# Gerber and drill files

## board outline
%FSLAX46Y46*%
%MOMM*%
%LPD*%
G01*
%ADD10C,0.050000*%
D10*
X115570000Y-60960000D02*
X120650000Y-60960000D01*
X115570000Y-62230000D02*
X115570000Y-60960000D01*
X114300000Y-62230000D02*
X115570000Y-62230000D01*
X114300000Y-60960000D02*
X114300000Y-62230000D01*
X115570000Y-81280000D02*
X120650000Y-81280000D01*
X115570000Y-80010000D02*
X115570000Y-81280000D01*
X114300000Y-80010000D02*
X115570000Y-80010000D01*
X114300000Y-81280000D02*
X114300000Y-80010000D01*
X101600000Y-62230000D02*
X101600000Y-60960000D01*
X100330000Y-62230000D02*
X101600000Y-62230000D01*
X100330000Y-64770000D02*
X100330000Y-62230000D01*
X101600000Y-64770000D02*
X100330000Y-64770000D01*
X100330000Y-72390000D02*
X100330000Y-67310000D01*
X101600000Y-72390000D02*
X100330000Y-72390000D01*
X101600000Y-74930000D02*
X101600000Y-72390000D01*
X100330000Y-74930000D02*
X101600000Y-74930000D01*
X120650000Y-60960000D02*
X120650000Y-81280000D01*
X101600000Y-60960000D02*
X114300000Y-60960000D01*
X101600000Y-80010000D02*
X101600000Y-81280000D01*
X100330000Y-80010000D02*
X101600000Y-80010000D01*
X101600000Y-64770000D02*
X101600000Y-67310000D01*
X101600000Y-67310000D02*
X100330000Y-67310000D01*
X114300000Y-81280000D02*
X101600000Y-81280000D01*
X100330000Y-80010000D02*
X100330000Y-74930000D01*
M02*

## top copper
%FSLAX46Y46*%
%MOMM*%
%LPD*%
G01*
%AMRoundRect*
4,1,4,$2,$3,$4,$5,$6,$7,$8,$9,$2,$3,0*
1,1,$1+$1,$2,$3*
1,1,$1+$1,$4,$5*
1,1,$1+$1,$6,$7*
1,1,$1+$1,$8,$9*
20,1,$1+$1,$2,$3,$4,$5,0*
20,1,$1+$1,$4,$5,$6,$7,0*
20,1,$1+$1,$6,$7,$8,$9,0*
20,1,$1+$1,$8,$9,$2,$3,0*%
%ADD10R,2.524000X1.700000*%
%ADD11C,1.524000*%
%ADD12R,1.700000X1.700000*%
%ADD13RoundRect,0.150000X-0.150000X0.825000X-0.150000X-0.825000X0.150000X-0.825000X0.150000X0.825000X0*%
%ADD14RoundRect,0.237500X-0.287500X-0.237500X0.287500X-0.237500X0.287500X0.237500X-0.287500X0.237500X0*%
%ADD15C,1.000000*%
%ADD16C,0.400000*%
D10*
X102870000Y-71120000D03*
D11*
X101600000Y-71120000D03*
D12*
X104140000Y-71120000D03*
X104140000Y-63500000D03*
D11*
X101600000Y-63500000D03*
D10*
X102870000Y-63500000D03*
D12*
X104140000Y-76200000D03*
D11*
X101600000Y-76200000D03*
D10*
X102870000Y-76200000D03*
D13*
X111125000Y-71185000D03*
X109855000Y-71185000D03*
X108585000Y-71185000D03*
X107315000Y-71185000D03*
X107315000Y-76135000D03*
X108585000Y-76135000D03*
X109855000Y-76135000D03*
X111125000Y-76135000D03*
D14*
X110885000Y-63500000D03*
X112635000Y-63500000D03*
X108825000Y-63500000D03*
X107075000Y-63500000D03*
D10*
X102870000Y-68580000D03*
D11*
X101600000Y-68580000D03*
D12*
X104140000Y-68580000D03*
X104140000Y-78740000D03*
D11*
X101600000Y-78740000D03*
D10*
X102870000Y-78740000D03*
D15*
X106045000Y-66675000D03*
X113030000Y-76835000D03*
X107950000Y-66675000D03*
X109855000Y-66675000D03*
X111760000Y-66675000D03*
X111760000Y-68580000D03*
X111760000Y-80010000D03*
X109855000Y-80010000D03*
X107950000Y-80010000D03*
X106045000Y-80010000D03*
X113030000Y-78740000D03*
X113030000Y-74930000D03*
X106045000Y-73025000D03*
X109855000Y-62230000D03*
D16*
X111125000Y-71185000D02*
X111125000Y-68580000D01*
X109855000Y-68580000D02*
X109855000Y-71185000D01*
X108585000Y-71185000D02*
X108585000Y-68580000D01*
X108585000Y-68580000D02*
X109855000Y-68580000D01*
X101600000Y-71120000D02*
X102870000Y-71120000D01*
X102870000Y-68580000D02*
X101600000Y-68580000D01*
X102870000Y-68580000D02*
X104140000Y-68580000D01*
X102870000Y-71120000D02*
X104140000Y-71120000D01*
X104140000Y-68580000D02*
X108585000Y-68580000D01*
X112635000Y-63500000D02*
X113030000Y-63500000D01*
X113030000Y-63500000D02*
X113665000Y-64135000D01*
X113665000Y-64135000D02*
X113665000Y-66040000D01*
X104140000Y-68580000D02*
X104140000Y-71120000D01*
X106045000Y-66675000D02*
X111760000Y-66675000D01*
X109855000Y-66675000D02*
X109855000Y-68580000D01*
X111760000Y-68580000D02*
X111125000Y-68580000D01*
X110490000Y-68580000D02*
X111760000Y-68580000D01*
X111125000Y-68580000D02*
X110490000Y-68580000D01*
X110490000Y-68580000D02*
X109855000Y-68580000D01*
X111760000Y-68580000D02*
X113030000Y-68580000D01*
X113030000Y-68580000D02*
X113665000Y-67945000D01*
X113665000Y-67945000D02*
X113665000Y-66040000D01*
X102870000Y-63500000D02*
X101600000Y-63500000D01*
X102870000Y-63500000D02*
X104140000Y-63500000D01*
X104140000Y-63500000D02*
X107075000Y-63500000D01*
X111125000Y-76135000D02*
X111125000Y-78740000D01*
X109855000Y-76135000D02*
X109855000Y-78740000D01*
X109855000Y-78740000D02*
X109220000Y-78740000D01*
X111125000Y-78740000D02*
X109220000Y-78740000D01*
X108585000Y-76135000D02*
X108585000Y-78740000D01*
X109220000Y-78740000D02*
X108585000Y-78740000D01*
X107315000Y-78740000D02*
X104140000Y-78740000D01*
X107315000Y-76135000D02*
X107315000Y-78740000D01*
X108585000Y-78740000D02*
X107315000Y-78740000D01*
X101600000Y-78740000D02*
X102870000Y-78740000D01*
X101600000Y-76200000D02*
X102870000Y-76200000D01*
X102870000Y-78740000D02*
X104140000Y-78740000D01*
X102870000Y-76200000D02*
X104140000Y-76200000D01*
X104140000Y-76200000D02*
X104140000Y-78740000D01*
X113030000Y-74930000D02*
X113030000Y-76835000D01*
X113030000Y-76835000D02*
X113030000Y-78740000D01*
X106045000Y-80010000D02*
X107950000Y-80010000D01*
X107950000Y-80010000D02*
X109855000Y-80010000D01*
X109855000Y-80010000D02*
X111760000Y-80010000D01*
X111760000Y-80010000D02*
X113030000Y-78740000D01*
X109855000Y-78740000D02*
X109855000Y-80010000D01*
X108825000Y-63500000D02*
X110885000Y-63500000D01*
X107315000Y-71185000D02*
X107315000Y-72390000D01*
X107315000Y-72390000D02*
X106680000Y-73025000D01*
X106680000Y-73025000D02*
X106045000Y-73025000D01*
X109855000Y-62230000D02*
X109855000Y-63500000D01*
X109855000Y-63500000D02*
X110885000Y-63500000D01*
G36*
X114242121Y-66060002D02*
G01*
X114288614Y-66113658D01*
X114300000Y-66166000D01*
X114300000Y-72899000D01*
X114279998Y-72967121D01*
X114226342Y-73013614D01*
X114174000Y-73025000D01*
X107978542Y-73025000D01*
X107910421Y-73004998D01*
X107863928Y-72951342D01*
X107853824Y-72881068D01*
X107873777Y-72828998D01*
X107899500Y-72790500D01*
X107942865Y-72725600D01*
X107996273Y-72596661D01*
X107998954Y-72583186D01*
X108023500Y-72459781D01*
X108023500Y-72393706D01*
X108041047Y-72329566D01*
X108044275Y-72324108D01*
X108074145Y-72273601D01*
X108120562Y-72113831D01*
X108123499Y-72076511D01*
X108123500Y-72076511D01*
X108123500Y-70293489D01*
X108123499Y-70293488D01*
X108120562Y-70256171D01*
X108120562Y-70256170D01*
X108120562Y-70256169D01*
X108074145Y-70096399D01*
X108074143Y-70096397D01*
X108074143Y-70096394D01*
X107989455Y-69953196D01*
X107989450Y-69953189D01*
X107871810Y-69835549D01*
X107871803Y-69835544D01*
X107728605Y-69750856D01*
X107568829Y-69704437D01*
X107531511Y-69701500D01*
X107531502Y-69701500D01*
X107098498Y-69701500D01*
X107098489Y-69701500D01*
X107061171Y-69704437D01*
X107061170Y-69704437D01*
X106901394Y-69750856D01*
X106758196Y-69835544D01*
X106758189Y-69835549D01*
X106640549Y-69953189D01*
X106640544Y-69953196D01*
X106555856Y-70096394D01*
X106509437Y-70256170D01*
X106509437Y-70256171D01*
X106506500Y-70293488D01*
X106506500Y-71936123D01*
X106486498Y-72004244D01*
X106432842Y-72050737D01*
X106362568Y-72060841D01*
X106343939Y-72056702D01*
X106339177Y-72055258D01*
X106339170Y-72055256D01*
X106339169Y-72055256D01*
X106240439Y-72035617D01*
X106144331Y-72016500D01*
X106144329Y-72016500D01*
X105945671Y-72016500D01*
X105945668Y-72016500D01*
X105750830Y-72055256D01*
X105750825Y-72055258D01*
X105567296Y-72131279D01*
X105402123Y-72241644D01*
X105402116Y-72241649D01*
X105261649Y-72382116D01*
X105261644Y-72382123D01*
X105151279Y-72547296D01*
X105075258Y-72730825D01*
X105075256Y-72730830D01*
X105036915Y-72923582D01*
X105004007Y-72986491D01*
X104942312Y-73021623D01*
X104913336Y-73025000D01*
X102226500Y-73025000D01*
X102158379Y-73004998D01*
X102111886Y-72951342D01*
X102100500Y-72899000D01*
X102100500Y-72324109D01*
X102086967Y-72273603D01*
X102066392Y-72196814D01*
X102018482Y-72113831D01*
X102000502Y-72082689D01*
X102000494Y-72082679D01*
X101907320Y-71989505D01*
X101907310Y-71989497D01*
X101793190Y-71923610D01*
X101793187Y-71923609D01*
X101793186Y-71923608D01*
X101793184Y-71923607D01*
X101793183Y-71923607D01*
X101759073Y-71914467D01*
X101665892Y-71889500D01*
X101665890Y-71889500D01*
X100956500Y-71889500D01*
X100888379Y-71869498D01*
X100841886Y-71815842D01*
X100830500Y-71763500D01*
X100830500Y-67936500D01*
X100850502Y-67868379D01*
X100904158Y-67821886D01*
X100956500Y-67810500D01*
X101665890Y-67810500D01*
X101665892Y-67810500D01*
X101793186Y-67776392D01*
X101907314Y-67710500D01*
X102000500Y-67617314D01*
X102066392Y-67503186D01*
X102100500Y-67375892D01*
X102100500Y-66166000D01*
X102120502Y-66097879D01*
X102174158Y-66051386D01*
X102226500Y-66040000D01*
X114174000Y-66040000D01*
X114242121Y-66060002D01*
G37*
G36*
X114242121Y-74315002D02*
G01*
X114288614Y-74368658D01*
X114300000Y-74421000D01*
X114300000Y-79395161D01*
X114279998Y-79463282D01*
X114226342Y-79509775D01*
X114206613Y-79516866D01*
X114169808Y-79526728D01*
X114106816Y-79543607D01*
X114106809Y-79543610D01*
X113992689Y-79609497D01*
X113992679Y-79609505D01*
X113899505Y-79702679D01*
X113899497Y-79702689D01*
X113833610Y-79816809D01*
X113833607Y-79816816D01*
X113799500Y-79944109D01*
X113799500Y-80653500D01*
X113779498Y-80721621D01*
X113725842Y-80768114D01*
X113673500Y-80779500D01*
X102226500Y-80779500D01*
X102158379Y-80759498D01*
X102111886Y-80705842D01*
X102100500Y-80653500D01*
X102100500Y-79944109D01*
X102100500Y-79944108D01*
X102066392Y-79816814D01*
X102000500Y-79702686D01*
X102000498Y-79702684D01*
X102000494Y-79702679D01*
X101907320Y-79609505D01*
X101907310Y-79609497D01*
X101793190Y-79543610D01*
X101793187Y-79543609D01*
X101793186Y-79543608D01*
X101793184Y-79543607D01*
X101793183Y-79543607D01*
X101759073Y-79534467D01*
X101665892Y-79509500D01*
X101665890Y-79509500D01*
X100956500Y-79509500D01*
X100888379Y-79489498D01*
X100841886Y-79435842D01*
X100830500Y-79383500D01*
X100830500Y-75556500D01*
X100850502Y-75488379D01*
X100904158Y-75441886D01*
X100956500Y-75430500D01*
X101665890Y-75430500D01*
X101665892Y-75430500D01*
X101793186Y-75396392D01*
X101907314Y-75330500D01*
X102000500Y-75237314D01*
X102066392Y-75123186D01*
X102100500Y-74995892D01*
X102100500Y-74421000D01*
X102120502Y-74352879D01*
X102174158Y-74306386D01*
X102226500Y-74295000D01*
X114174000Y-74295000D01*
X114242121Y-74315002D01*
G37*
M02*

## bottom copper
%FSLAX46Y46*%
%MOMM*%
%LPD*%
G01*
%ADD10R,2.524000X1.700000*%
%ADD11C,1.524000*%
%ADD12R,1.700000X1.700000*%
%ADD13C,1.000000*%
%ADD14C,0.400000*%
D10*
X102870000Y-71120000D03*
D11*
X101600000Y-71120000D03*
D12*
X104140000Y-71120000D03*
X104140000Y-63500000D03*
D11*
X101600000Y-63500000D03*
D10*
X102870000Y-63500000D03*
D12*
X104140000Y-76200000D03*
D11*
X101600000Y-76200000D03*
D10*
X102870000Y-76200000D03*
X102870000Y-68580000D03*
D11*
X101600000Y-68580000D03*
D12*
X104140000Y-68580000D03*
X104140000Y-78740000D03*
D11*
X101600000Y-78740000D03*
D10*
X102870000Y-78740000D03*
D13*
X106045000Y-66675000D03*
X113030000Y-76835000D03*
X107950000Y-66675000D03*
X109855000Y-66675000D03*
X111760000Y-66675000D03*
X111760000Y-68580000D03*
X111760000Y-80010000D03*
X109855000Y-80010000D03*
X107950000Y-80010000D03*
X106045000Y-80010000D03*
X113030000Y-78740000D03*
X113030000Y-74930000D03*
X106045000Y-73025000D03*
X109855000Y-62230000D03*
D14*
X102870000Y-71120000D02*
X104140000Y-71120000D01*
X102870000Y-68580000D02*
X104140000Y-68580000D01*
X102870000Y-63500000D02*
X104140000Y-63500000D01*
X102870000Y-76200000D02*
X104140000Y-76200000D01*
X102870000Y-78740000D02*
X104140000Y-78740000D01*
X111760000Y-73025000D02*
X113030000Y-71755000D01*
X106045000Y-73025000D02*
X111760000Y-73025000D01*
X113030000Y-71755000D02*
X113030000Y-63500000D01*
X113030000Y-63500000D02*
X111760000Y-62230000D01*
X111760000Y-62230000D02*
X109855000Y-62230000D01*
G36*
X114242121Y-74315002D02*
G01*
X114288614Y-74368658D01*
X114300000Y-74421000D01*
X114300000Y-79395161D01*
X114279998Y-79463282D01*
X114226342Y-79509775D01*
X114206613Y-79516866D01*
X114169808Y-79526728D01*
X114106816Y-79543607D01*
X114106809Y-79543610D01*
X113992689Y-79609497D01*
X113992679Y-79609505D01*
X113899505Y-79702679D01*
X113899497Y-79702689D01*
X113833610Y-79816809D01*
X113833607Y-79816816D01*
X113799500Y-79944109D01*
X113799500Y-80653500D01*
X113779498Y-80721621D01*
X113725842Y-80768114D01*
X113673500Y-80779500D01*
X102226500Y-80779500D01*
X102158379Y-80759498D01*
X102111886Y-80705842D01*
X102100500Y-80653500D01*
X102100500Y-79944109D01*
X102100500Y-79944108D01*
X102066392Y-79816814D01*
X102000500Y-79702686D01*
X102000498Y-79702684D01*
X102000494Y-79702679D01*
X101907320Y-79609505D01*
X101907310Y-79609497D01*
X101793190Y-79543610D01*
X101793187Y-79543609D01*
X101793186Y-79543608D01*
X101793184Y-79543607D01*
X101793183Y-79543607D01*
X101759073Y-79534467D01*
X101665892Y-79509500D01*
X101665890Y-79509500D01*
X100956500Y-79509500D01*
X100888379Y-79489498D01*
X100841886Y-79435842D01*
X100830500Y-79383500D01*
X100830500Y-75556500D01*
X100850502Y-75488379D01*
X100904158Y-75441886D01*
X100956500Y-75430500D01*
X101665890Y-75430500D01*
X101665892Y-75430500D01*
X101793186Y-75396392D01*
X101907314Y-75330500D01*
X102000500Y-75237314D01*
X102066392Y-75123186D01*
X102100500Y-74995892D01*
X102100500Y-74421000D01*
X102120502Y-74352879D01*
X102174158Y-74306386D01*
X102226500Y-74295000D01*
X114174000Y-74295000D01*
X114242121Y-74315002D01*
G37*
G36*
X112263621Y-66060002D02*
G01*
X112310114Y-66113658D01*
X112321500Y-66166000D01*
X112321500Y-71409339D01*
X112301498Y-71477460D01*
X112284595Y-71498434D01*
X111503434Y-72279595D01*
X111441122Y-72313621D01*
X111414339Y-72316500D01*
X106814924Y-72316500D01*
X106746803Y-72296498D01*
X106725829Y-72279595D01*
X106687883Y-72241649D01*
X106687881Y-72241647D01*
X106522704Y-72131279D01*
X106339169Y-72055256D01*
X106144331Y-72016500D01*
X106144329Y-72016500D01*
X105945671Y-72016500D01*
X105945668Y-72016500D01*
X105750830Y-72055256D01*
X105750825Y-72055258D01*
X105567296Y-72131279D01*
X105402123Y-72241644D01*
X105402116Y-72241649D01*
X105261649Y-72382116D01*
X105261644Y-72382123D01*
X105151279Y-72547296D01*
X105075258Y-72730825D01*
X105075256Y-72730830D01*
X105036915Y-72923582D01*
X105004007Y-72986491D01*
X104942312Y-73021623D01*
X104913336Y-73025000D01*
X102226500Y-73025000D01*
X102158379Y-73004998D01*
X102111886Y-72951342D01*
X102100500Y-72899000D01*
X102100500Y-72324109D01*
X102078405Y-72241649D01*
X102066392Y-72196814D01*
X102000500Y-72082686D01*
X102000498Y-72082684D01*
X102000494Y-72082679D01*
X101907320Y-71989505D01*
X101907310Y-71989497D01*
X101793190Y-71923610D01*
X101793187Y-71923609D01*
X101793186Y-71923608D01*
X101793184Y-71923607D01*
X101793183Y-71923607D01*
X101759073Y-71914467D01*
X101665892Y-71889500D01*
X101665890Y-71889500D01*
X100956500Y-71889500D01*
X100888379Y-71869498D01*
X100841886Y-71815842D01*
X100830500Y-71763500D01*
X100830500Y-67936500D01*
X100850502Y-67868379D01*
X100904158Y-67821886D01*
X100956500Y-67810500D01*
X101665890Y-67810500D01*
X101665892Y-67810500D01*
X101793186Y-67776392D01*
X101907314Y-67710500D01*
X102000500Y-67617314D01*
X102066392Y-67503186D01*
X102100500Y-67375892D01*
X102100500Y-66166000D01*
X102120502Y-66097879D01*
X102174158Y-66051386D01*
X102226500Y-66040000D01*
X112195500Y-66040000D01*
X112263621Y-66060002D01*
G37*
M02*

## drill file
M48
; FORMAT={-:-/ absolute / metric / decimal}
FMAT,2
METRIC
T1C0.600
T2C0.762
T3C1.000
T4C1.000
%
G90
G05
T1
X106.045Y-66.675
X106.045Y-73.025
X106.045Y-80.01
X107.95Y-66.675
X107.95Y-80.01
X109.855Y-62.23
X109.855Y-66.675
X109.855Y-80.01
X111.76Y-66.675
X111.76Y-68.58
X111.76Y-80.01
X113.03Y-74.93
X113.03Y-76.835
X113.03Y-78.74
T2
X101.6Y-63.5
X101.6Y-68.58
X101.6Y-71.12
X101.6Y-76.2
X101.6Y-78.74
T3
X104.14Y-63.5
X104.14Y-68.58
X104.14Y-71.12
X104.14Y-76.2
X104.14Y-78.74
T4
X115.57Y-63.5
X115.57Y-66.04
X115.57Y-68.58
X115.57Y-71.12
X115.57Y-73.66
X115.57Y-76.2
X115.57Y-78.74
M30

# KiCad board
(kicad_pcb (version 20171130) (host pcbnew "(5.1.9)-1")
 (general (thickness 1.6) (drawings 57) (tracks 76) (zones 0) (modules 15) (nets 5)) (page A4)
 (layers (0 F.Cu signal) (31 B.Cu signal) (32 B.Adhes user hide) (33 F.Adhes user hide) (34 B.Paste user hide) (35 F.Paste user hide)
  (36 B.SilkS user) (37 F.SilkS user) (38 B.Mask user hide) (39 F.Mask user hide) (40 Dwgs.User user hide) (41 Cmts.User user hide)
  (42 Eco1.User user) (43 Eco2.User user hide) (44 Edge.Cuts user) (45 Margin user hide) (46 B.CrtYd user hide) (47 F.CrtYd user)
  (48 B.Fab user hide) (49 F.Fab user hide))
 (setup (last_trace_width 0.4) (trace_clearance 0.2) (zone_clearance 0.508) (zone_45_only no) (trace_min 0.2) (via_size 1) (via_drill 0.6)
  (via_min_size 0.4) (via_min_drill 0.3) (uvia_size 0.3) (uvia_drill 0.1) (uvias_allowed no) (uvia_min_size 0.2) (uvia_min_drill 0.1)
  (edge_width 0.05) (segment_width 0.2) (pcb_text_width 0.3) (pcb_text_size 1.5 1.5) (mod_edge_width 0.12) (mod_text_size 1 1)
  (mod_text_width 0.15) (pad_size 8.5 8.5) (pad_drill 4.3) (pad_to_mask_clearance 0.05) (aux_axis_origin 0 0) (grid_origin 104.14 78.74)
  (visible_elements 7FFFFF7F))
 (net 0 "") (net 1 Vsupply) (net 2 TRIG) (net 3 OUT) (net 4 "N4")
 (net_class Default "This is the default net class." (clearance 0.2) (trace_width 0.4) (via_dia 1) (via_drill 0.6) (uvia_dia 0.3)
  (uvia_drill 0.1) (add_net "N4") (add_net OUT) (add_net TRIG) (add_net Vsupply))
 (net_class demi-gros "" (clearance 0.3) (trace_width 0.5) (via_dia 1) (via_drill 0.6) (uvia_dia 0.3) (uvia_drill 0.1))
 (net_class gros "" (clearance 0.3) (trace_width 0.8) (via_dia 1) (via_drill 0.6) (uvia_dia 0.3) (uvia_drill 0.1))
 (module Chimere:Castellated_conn (layer F.Cu) (at 104.14 71.12 180)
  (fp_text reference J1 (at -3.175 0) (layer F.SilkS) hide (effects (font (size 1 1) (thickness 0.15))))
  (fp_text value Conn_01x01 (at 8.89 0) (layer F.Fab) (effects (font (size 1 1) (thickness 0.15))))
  (pad 1 smd rect (at 1.27 0 180) (size 2.524 1.7) (layers B.Cu F.Paste F.Mask) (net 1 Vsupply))
  (pad 1 smd rect (at 1.27 0 180) (size 2.524 1.7) (layers F.Cu F.Paste F.Mask) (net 1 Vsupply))
  (pad 1 thru_hole circle (at 2.54 0 180) (size 1.524 1.524) (drill 0.762) (layers *.Cu *.Mask) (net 1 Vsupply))
  (pad 1 thru_hole rect (at 0 0 180) (size 1.7 1.7) (drill 1) (layers *.Cu *.Mask) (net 1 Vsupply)))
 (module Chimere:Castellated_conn (layer F.Cu) (at 104.14 63.5 180)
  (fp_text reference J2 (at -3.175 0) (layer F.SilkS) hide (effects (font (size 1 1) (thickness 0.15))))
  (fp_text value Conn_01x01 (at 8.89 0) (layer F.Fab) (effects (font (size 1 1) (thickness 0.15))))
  (pad 1 thru_hole rect (at 0 0 180) (size 1.7 1.7) (drill 1) (layers *.Cu *.Mask) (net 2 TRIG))
  (pad 1 thru_hole circle (at 2.54 0 180) (size 1.524 1.524) (drill 0.762) (layers *.Cu *.Mask) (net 2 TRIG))
  (pad 1 smd rect (at 1.27 0 180) (size 2.524 1.7) (layers F.Cu F.Paste F.Mask) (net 2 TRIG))
  (pad 1 smd rect (at 1.27 0 180) (size 2.524 1.7) (layers B.Cu F.Paste F.Mask) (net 2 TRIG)))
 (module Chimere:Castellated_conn (layer F.Cu) (at 104.14 76.2 180)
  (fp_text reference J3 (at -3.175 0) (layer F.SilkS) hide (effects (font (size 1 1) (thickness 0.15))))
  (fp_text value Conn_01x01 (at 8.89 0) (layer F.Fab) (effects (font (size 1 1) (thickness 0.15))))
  (pad 1 thru_hole rect (at 0 0 180) (size 1.7 1.7) (drill 1) (layers *.Cu *.Mask) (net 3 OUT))
  (pad 1 thru_hole circle (at 2.54 0 180) (size 1.524 1.524) (drill 0.762) (layers *.Cu *.Mask) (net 3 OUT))
  (pad 1 smd rect (at 1.27 0 180) (size 2.524 1.7) (layers F.Cu F.Paste F.Mask) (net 3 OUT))
  (pad 1 smd rect (at 1.27 0 180) (size 2.524 1.7) (layers B.Cu F.Paste F.Mask) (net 3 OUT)))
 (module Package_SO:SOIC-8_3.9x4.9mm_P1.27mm (layer F.Cu) (at 109.22 73.66 270)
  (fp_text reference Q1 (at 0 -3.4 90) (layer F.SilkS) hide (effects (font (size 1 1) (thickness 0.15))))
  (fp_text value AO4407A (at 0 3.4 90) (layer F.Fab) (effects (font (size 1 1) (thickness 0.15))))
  (pad 1 smd roundrect (at -2.475 -1.905 270) (size 1.95 0.6) (layers F.Cu F.Paste F.Mask) (roundrect_rratio 0.25) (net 1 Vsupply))
  (pad 2 smd roundrect (at -2.475 -0.635 270) (size 1.95 0.6) (layers F.Cu F.Paste F.Mask) (roundrect_rratio 0.25) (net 1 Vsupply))
  (pad 3 smd roundrect (at -2.475 0.635 270) (size 1.95 0.6) (layers F.Cu F.Paste F.Mask) (roundrect_rratio 0.25) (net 1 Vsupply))
  (pad 4 smd roundrect (at -2.475 1.905 270) (size 1.95 0.6) (layers F.Cu F.Paste F.Mask) (roundrect_rratio 0.25) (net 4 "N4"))
  (pad 5 smd roundrect (at 2.475 1.905 270) (size 1.95 0.6) (layers F.Cu F.Paste F.Mask) (roundrect_rratio 0.25) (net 3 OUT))
  (pad 6 smd roundrect (at 2.475 0.635 270) (size 1.95 0.6) (layers F.Cu F.Paste F.Mask) (roundrect_rratio 0.25) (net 3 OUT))
  (pad 7 smd roundrect (at 2.475 -0.635 270) (size 1.95 0.6) (layers F.Cu F.Paste F.Mask) (roundrect_rratio 0.25) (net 3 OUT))
  (pad 8 smd roundrect (at 2.475 -1.905 270) (size 1.95 0.6) (layers F.Cu F.Paste F.Mask) (roundrect_rratio 0.25) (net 3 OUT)))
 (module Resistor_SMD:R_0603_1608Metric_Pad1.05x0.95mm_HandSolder (layer F.Cu) (at 111.76 63.5)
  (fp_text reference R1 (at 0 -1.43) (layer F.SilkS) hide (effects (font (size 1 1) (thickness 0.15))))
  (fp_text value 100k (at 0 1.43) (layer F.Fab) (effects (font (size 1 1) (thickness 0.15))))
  (pad 1 smd roundrect (at -0.875 0) (size 1.05 0.95) (layers F.Cu F.Paste F.Mask) (roundrect_rratio 0.25) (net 4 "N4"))
  (pad 2 smd roundrect (at 0.875 0) (size 1.05 0.95) (layers F.Cu F.Paste F.Mask) (roundrect_rratio 0.25) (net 1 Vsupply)))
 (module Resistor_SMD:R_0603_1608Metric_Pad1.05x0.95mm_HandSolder (layer F.Cu) (at 107.95 63.5)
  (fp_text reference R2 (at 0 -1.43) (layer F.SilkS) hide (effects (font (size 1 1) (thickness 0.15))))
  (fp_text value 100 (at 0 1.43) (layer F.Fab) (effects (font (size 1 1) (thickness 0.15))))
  (pad 2 smd roundrect (at 0.875 0) (size 1.05 0.95) (layers F.Cu F.Paste F.Mask) (roundrect_rratio 0.25) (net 4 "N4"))
  (pad 1 smd roundrect (at -0.875 0) (size 1.05 0.95) (layers F.Cu F.Paste F.Mask) (roundrect_rratio 0.25) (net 2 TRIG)))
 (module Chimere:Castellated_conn (layer F.Cu) (at 104.14 68.58 180)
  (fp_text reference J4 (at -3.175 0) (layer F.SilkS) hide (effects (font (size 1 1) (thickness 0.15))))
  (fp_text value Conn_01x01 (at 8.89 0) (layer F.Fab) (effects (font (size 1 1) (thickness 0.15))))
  (pad 1 smd rect (at 1.27 0 180) (size 2.524 1.7) (layers B.Cu F.Paste F.Mask) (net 1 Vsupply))
  (pad 1 smd rect (at 1.27 0 180) (size 2.524 1.7) (layers F.Cu F.Paste F.Mask) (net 1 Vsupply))
  (pad 1 thru_hole circle (at 2.54 0 180) (size 1.524 1.524) (drill 0.762) (layers *.Cu *.Mask) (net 1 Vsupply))
  (pad 1 thru_hole rect (at 0 0 180) (size 1.7 1.7) (drill 1) (layers *.Cu *.Mask) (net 1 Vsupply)))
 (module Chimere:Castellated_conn (layer F.Cu) (at 104.14 78.74 180)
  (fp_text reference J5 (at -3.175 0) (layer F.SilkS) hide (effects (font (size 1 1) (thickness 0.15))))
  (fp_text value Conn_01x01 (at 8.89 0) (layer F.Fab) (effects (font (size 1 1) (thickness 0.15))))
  (pad 1 thru_hole rect (at 0 0 180) (size 1.7 1.7) (drill 1) (layers *.Cu *.Mask) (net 3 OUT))
  (pad 1 thru_hole circle (at 2.54 0 180) (size 1.524 1.524) (drill 0.762) (layers *.Cu *.Mask) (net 3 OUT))
  (pad 1 smd rect (at 1.27 0 180) (size 2.524 1.7) (layers F.Cu F.Paste F.Mask) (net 3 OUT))
  (pad 1 smd rect (at 1.27 0 180) (size 2.524 1.7) (layers B.Cu F.Paste F.Mask) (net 3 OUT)))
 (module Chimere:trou (layer F.Cu) (at 115.57 63.5)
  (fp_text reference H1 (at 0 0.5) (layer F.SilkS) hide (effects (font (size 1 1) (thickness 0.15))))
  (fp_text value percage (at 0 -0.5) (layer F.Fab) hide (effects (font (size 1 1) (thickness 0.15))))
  (pad "" np_thru_hole circle (at 0 0) (size 1 1) (drill 1) (layers *.Cu *.Mask)))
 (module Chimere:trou (layer F.Cu) (at 115.57 66.04)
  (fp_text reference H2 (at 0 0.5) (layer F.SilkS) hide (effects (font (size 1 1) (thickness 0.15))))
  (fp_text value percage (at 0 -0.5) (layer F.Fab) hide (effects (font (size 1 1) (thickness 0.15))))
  (pad "" np_thru_hole circle (at 0 0) (size 1 1) (drill 1) (layers *.Cu *.Mask)))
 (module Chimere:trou (layer F.Cu) (at 115.57 78.74)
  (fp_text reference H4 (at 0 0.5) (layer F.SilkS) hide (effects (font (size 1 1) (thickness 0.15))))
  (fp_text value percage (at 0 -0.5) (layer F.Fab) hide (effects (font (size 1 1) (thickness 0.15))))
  (pad "" np_thru_hole circle (at 0 0) (size 1 1) (drill 1) (layers *.Cu *.Mask)))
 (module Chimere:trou (layer F.Cu) (at 115.57 71.12)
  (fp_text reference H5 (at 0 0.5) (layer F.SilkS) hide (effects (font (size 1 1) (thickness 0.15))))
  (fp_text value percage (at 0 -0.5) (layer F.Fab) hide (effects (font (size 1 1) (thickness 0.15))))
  (pad "" np_thru_hole circle (at 0 0) (size 1 1) (drill 1) (layers *.Cu *.Mask)))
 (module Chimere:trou (layer F.Cu) (at 115.57 76.2)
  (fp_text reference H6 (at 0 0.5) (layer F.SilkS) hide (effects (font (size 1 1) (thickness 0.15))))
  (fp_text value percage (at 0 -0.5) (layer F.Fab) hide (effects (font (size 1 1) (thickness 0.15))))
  (pad "" np_thru_hole circle (at 0 0) (size 1 1) (drill 1) (layers *.Cu *.Mask)))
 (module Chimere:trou (layer F.Cu) (at 115.57 68.58)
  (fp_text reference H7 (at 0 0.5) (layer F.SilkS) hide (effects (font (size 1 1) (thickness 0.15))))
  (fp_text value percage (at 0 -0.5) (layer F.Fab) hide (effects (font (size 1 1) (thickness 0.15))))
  (pad "" np_thru_hole circle (at 0 0) (size 1 1) (drill 1) (layers *.Cu *.Mask)))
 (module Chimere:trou (layer F.Cu) (at 115.57 73.66)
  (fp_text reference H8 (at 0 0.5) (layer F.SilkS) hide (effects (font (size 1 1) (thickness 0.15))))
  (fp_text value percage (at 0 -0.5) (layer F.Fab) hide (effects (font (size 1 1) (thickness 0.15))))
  (pad "" np_thru_hole circle (at 0 0) (size 1 1) (drill 1) (layers *.Cu *.Mask)))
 (gr_line (start 115.57 60.96) (end 120.65 60.96) (layer Edge.Cuts) (width 0.05))
 (gr_line (start 115.57 62.23) (end 115.57 60.96) (layer Edge.Cuts) (width 0.05))
 (gr_line (start 114.3 62.23) (end 115.57 62.23) (layer Edge.Cuts) (width 0.05))
 (gr_line (start 114.3 60.96) (end 114.3 62.23) (layer Edge.Cuts) (width 0.05))
 (gr_line (start 115.57 81.28) (end 120.65 81.28) (layer Edge.Cuts) (width 0.05))
 (gr_line (start 115.57 80.01) (end 115.57 81.28) (layer Edge.Cuts) (width 0.05))
 (gr_line (start 114.3 80.01) (end 115.57 80.01) (layer Edge.Cuts) (width 0.05))
 (gr_line (start 114.3 81.28) (end 114.3 80.01) (layer Edge.Cuts) (width 0.05))
 (gr_line (start 101.6 62.23) (end 101.6 60.96) (layer Edge.Cuts) (width 0.05))
 (gr_line (start 100.33 62.23) (end 101.6 62.23) (layer Edge.Cuts) (width 0.05))
 (gr_line (start 100.33 64.77) (end 100.33 62.23) (layer Edge.Cuts) (width 0.05))
 (gr_line (start 101.6 64.77) (end 100.33 64.77) (layer Edge.Cuts) (width 0.05))
 (gr_line (start 100.33 72.39) (end 100.33 67.31) (layer Edge.Cuts) (width 0.05))
 (gr_line (start 101.6 72.39) (end 100.33 72.39) (layer Edge.Cuts) (width 0.05))
 (gr_line (start 101.6 74.93) (end 101.6 72.39) (layer Edge.Cuts) (width 0.05))
 (gr_line (start 100.33 74.93) (end 101.6 74.93) (layer Edge.Cuts) (width 0.05))
 (gr_line (start 120.65 60.96) (end 120.65 81.28) (layer Edge.Cuts) (width 0.05))
 (gr_line (start 101.6 60.96) (end 114.3 60.96) (layer Edge.Cuts) (width 0.05))
 (gr_line (start 101.6 80.01) (end 101.6 81.28) (layer Edge.Cuts) (width 0.05))
 (gr_line (start 100.33 80.01) (end 101.6 80.01) (layer Edge.Cuts) (width 0.05))
 (gr_line (start 101.6 64.77) (end 101.6 67.31) (layer Edge.Cuts) (width 0.05))
 (gr_line (start 101.6 67.31) (end 100.33 67.31) (layer Edge.Cuts) (width 0.05))
 (gr_line (start 114.3 81.28) (end 101.6 81.28) (layer Edge.Cuts) (width 0.05))
 (gr_line (start 100.33 80.01) (end 100.33 74.93) (layer Edge.Cuts) (width 0.05))
 (via (at 106.045 66.675) (size 1) (drill 0.6) (layers F.Cu B.Cu) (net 1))
 (via (at 113.03 76.835) (size 1) (drill 0.6) (layers F.Cu B.Cu) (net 3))
 (segment (start 111.125 71.185) (end 111.125 68.58) (width 0.4) (layer F.Cu) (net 1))
 (segment (start 109.855 68.58) (end 109.855 71.185) (width 0.4) (layer F.Cu) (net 1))
 (segment (start 108.585 71.185) (end 108.585 68.58) (width 0.4) (layer F.Cu) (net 1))
 (segment (start 108.585 68.58) (end 109.855 68.58) (width 0.4) (layer F.Cu) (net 1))
 (segment (start 102.87 71.12) (end 104.14 71.12) (width 0.4) (layer B.Cu) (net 1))
 (segment (start 102.87 68.58) (end 104.14 68.58) (width 0.4) (layer B.Cu) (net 1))
 (segment (start 101.6 71.12) (end 102.87 71.12) (width 0.4) (layer F.Cu) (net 1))
 (segment (start 102.87 68.58) (end 101.6 68.58) (width 0.4) (layer F.Cu) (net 1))
 (segment (start 102.87 68.58) (end 104.14 68.58) (width 0.4) (layer F.Cu) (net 1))
 (segment (start 102.87 71.12) (end 104.14 71.12) (width 0.4) (layer F.Cu) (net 1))
 (segment (start 104.14 68.58) (end 108.585 68.58) (width 0.4) (layer F.Cu) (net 1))
 (segment (start 112.635 63.5) (end 113.03 63.5) (width 0.4) (layer F.Cu) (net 1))
 (segment (start 113.03 63.5) (end 113.665 64.135) (width 0.4) (layer F.Cu) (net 1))
 (segment (start 113.665 64.135) (end 113.665 66.04) (width 0.4) (layer F.Cu) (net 1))
 (segment (start 104.14 68.58) (end 104.14 71.12) (width 0.4) (layer F.Cu) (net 1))
 (via (at 107.95 66.675) (size 1) (drill 0.6) (layers F.Cu B.Cu) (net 1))
 (via (at 109.855 66.675) (size 1) (drill 0.6) (layers F.Cu B.Cu) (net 1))
 (via (at 111.76 66.675) (size 1) (drill 0.6) (layers F.Cu B.Cu) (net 1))
 (via (at 111.76 68.58) (size 1) (drill 0.6) (layers F.Cu B.Cu) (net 1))
 (segment (start 106.045 66.675) (end 111.76 66.675) (width 0.4) (layer F.Cu) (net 1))
 (segment (start 109.855 66.675) (end 109.855 68.58) (width 0.4) (layer F.Cu) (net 1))
 (segment (start 111.76 68.58) (end 111.125 68.58) (width 0.4) (layer F.Cu) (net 1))
 (segment (start 110.49 68.58) (end 111.76 68.58) (width 0.4) (layer F.Cu) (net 1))
 (segment (start 111.125 68.58) (end 110.49 68.58) (width 0.4) (layer F.Cu) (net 1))
 (segment (start 110.49 68.58) (end 109.855 68.58) (width 0.4) (layer F.Cu) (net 1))
 (segment (start 111.76 68.58) (end 113.03 68.58) (width 0.4) (layer F.Cu) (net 1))
 (segment (start 113.03 68.58) (end 113.665 67.945) (width 0.4) (layer F.Cu) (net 1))
 (segment (start 113.665 67.945) (end 113.665 66.04) (width 0.4) (layer F.Cu) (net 1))
 (segment (start 102.87 63.5) (end 104.14 63.5) (width 0.4) (layer B.Cu) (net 2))
 (segment (start 102.87 63.5) (end 101.6 63.5) (width 0.4) (layer F.Cu) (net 2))
 (segment (start 102.87 63.5) (end 104.14 63.5) (width 0.4) (layer F.Cu) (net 2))
 (segment (start 104.14 63.5) (end 107.075 63.5) (width 0.4) (layer F.Cu) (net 2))
 (segment (start 111.125 76.135) (end 111.125 78.74) (width 0.4) (layer F.Cu) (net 3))
 (segment (start 109.855 76.135) (end 109.855 78.74) (width 0.4) (layer F.Cu) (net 3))
 (segment (start 109.855 78.74) (end 109.22 78.74) (width 0.4) (layer F.Cu) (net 3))
 (segment (start 111.125 78.74) (end 109.22 78.74) (width 0.4) (layer F.Cu) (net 3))
 (segment (start 108.585 76.135) (end 108.585 78.74) (width 0.4) (layer F.Cu) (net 3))
 (segment (start 109.22 78.74) (end 108.585 78.74) (width 0.4) (layer F.Cu) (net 3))
 (segment (start 107.315 78.74) (end 104.14 78.74) (width 0.4) (layer F.Cu) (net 3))
 (segment (start 107.315 76.135) (end 107.315 78.74) (width 0.4) (layer F.Cu) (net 3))
 (segment (start 108.585 78.74) (end 107.315 78.74) (width 0.4) (layer F.Cu) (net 3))
 (segment (start 101.6 78.74) (end 102.87 78.74) (width 0.4) (layer F.Cu) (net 3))
 (segment (start 101.6 76.2) (end 102.87 76.2) (width 0.4) (layer F.Cu) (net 3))
 (segment (start 102.87 78.74) (end 104.14 78.74) (width 0.4) (layer F.Cu) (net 3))
 (segment (start 102.87 76.2) (end 104.14 76.2) (width 0.4) (layer B.Cu) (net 3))
 (segment (start 102.87 78.74) (end 104.14 78.74) (width 0.4) (layer B.Cu) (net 3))
 (segment (start 102.87 76.2) (end 104.14 76.2) (width 0.4) (layer F.Cu) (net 3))
 (segment (start 104.14 76.2) (end 104.14 78.74) (width 0.4) (layer F.Cu) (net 3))
 (via (at 111.76 80.01) (size 1) (drill 0.6) (layers F.Cu B.Cu) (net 3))
 (via (at 109.855 80.01) (size 1) (drill 0.6) (layers F.Cu B.Cu) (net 3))
 (via (at 107.95 80.01) (size 1) (drill 0.6) (layers F.Cu B.Cu) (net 3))
 (via (at 106.045 80.01) (size 1) (drill 0.6) (layers F.Cu B.Cu) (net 3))
 (via (at 113.03 78.74) (size 1) (drill 0.6) (layers F.Cu B.Cu) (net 3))
 (via (at 113.03 74.93) (size 1) (drill 0.6) (layers F.Cu B.Cu) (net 3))
 (segment (start 113.03 74.93) (end 113.03 76.835) (width 0.4) (layer F.Cu) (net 3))
 (segment (start 113.03 76.835) (end 113.03 78.74) (width 0.4) (layer F.Cu) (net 3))
 (segment (start 106.045 80.01) (end 107.95 80.01) (width 0.4) (layer F.Cu) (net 3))
 (segment (start 107.95 80.01) (end 109.855 80.01) (width 0.4) (layer F.Cu) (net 3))
 (segment (start 109.855 80.01) (end 111.76 80.01) (width 0.4) (layer F.Cu) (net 3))
 (segment (start 111.76 80.01) (end 113.03 78.74) (width 0.4) (layer F.Cu) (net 3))
 (segment (start 109.855 78.74) (end 109.855 80.01) (width 0.4) (layer F.Cu) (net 3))
 (segment (start 108.825 63.5) (end 110.885 63.5) (width 0.4) (layer F.Cu) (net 4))
 (segment (start 107.315 71.185) (end 107.315 72.39) (width 0.4) (layer F.Cu) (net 4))
 (segment (start 107.315 72.39) (end 106.68 73.025) (width 0.4) (layer F.Cu) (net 4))
 (via (at 106.045 73.025) (size 1) (drill 0.6) (layers F.Cu B.Cu) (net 4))
 (segment (start 106.68 73.025) (end 106.045 73.025) (width 0.4) (layer F.Cu) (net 4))
 (via (at 109.855 62.23) (size 1) (drill 0.6) (layers F.Cu B.Cu) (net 4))
 (segment (start 109.855 62.23) (end 109.855 63.5) (width 0.4) (layer F.Cu) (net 4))
 (segment (start 109.855 63.5) (end 110.885 63.5) (width 0.4) (layer F.Cu) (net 4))
 (segment (start 111.76 73.025) (end 113.03 71.755) (width 0.4) (layer B.Cu) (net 4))
 (segment (start 106.045 73.025) (end 111.76 73.025) (width 0.4) (layer B.Cu) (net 4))
 (segment (start 113.03 71.755) (end 113.03 63.5) (width 0.4) (layer B.Cu) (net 4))
 (segment (start 113.03 63.5) (end 111.76 62.23) (width 0.4) (layer B.Cu) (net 4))
 (segment (start 111.76 62.23) (end 109.855 62.23) (width 0.4) (layer B.Cu) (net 4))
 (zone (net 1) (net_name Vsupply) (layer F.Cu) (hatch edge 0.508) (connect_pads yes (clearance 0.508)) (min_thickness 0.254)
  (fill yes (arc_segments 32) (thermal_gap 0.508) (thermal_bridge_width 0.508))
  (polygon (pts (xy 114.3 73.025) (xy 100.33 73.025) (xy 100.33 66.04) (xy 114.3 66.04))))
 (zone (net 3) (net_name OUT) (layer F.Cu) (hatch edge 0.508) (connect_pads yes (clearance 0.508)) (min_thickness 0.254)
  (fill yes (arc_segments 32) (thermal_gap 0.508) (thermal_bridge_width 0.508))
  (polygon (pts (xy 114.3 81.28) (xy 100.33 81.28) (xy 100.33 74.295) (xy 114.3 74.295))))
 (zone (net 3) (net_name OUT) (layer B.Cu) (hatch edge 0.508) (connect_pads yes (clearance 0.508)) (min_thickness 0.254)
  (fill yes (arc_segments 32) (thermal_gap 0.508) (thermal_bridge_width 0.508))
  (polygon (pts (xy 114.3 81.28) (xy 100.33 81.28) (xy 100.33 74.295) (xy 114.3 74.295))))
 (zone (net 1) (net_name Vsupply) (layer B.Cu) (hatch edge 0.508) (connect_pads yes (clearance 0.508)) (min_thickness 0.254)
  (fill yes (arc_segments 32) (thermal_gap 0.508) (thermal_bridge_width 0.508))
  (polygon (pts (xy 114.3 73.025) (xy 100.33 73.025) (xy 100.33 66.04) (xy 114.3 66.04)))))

